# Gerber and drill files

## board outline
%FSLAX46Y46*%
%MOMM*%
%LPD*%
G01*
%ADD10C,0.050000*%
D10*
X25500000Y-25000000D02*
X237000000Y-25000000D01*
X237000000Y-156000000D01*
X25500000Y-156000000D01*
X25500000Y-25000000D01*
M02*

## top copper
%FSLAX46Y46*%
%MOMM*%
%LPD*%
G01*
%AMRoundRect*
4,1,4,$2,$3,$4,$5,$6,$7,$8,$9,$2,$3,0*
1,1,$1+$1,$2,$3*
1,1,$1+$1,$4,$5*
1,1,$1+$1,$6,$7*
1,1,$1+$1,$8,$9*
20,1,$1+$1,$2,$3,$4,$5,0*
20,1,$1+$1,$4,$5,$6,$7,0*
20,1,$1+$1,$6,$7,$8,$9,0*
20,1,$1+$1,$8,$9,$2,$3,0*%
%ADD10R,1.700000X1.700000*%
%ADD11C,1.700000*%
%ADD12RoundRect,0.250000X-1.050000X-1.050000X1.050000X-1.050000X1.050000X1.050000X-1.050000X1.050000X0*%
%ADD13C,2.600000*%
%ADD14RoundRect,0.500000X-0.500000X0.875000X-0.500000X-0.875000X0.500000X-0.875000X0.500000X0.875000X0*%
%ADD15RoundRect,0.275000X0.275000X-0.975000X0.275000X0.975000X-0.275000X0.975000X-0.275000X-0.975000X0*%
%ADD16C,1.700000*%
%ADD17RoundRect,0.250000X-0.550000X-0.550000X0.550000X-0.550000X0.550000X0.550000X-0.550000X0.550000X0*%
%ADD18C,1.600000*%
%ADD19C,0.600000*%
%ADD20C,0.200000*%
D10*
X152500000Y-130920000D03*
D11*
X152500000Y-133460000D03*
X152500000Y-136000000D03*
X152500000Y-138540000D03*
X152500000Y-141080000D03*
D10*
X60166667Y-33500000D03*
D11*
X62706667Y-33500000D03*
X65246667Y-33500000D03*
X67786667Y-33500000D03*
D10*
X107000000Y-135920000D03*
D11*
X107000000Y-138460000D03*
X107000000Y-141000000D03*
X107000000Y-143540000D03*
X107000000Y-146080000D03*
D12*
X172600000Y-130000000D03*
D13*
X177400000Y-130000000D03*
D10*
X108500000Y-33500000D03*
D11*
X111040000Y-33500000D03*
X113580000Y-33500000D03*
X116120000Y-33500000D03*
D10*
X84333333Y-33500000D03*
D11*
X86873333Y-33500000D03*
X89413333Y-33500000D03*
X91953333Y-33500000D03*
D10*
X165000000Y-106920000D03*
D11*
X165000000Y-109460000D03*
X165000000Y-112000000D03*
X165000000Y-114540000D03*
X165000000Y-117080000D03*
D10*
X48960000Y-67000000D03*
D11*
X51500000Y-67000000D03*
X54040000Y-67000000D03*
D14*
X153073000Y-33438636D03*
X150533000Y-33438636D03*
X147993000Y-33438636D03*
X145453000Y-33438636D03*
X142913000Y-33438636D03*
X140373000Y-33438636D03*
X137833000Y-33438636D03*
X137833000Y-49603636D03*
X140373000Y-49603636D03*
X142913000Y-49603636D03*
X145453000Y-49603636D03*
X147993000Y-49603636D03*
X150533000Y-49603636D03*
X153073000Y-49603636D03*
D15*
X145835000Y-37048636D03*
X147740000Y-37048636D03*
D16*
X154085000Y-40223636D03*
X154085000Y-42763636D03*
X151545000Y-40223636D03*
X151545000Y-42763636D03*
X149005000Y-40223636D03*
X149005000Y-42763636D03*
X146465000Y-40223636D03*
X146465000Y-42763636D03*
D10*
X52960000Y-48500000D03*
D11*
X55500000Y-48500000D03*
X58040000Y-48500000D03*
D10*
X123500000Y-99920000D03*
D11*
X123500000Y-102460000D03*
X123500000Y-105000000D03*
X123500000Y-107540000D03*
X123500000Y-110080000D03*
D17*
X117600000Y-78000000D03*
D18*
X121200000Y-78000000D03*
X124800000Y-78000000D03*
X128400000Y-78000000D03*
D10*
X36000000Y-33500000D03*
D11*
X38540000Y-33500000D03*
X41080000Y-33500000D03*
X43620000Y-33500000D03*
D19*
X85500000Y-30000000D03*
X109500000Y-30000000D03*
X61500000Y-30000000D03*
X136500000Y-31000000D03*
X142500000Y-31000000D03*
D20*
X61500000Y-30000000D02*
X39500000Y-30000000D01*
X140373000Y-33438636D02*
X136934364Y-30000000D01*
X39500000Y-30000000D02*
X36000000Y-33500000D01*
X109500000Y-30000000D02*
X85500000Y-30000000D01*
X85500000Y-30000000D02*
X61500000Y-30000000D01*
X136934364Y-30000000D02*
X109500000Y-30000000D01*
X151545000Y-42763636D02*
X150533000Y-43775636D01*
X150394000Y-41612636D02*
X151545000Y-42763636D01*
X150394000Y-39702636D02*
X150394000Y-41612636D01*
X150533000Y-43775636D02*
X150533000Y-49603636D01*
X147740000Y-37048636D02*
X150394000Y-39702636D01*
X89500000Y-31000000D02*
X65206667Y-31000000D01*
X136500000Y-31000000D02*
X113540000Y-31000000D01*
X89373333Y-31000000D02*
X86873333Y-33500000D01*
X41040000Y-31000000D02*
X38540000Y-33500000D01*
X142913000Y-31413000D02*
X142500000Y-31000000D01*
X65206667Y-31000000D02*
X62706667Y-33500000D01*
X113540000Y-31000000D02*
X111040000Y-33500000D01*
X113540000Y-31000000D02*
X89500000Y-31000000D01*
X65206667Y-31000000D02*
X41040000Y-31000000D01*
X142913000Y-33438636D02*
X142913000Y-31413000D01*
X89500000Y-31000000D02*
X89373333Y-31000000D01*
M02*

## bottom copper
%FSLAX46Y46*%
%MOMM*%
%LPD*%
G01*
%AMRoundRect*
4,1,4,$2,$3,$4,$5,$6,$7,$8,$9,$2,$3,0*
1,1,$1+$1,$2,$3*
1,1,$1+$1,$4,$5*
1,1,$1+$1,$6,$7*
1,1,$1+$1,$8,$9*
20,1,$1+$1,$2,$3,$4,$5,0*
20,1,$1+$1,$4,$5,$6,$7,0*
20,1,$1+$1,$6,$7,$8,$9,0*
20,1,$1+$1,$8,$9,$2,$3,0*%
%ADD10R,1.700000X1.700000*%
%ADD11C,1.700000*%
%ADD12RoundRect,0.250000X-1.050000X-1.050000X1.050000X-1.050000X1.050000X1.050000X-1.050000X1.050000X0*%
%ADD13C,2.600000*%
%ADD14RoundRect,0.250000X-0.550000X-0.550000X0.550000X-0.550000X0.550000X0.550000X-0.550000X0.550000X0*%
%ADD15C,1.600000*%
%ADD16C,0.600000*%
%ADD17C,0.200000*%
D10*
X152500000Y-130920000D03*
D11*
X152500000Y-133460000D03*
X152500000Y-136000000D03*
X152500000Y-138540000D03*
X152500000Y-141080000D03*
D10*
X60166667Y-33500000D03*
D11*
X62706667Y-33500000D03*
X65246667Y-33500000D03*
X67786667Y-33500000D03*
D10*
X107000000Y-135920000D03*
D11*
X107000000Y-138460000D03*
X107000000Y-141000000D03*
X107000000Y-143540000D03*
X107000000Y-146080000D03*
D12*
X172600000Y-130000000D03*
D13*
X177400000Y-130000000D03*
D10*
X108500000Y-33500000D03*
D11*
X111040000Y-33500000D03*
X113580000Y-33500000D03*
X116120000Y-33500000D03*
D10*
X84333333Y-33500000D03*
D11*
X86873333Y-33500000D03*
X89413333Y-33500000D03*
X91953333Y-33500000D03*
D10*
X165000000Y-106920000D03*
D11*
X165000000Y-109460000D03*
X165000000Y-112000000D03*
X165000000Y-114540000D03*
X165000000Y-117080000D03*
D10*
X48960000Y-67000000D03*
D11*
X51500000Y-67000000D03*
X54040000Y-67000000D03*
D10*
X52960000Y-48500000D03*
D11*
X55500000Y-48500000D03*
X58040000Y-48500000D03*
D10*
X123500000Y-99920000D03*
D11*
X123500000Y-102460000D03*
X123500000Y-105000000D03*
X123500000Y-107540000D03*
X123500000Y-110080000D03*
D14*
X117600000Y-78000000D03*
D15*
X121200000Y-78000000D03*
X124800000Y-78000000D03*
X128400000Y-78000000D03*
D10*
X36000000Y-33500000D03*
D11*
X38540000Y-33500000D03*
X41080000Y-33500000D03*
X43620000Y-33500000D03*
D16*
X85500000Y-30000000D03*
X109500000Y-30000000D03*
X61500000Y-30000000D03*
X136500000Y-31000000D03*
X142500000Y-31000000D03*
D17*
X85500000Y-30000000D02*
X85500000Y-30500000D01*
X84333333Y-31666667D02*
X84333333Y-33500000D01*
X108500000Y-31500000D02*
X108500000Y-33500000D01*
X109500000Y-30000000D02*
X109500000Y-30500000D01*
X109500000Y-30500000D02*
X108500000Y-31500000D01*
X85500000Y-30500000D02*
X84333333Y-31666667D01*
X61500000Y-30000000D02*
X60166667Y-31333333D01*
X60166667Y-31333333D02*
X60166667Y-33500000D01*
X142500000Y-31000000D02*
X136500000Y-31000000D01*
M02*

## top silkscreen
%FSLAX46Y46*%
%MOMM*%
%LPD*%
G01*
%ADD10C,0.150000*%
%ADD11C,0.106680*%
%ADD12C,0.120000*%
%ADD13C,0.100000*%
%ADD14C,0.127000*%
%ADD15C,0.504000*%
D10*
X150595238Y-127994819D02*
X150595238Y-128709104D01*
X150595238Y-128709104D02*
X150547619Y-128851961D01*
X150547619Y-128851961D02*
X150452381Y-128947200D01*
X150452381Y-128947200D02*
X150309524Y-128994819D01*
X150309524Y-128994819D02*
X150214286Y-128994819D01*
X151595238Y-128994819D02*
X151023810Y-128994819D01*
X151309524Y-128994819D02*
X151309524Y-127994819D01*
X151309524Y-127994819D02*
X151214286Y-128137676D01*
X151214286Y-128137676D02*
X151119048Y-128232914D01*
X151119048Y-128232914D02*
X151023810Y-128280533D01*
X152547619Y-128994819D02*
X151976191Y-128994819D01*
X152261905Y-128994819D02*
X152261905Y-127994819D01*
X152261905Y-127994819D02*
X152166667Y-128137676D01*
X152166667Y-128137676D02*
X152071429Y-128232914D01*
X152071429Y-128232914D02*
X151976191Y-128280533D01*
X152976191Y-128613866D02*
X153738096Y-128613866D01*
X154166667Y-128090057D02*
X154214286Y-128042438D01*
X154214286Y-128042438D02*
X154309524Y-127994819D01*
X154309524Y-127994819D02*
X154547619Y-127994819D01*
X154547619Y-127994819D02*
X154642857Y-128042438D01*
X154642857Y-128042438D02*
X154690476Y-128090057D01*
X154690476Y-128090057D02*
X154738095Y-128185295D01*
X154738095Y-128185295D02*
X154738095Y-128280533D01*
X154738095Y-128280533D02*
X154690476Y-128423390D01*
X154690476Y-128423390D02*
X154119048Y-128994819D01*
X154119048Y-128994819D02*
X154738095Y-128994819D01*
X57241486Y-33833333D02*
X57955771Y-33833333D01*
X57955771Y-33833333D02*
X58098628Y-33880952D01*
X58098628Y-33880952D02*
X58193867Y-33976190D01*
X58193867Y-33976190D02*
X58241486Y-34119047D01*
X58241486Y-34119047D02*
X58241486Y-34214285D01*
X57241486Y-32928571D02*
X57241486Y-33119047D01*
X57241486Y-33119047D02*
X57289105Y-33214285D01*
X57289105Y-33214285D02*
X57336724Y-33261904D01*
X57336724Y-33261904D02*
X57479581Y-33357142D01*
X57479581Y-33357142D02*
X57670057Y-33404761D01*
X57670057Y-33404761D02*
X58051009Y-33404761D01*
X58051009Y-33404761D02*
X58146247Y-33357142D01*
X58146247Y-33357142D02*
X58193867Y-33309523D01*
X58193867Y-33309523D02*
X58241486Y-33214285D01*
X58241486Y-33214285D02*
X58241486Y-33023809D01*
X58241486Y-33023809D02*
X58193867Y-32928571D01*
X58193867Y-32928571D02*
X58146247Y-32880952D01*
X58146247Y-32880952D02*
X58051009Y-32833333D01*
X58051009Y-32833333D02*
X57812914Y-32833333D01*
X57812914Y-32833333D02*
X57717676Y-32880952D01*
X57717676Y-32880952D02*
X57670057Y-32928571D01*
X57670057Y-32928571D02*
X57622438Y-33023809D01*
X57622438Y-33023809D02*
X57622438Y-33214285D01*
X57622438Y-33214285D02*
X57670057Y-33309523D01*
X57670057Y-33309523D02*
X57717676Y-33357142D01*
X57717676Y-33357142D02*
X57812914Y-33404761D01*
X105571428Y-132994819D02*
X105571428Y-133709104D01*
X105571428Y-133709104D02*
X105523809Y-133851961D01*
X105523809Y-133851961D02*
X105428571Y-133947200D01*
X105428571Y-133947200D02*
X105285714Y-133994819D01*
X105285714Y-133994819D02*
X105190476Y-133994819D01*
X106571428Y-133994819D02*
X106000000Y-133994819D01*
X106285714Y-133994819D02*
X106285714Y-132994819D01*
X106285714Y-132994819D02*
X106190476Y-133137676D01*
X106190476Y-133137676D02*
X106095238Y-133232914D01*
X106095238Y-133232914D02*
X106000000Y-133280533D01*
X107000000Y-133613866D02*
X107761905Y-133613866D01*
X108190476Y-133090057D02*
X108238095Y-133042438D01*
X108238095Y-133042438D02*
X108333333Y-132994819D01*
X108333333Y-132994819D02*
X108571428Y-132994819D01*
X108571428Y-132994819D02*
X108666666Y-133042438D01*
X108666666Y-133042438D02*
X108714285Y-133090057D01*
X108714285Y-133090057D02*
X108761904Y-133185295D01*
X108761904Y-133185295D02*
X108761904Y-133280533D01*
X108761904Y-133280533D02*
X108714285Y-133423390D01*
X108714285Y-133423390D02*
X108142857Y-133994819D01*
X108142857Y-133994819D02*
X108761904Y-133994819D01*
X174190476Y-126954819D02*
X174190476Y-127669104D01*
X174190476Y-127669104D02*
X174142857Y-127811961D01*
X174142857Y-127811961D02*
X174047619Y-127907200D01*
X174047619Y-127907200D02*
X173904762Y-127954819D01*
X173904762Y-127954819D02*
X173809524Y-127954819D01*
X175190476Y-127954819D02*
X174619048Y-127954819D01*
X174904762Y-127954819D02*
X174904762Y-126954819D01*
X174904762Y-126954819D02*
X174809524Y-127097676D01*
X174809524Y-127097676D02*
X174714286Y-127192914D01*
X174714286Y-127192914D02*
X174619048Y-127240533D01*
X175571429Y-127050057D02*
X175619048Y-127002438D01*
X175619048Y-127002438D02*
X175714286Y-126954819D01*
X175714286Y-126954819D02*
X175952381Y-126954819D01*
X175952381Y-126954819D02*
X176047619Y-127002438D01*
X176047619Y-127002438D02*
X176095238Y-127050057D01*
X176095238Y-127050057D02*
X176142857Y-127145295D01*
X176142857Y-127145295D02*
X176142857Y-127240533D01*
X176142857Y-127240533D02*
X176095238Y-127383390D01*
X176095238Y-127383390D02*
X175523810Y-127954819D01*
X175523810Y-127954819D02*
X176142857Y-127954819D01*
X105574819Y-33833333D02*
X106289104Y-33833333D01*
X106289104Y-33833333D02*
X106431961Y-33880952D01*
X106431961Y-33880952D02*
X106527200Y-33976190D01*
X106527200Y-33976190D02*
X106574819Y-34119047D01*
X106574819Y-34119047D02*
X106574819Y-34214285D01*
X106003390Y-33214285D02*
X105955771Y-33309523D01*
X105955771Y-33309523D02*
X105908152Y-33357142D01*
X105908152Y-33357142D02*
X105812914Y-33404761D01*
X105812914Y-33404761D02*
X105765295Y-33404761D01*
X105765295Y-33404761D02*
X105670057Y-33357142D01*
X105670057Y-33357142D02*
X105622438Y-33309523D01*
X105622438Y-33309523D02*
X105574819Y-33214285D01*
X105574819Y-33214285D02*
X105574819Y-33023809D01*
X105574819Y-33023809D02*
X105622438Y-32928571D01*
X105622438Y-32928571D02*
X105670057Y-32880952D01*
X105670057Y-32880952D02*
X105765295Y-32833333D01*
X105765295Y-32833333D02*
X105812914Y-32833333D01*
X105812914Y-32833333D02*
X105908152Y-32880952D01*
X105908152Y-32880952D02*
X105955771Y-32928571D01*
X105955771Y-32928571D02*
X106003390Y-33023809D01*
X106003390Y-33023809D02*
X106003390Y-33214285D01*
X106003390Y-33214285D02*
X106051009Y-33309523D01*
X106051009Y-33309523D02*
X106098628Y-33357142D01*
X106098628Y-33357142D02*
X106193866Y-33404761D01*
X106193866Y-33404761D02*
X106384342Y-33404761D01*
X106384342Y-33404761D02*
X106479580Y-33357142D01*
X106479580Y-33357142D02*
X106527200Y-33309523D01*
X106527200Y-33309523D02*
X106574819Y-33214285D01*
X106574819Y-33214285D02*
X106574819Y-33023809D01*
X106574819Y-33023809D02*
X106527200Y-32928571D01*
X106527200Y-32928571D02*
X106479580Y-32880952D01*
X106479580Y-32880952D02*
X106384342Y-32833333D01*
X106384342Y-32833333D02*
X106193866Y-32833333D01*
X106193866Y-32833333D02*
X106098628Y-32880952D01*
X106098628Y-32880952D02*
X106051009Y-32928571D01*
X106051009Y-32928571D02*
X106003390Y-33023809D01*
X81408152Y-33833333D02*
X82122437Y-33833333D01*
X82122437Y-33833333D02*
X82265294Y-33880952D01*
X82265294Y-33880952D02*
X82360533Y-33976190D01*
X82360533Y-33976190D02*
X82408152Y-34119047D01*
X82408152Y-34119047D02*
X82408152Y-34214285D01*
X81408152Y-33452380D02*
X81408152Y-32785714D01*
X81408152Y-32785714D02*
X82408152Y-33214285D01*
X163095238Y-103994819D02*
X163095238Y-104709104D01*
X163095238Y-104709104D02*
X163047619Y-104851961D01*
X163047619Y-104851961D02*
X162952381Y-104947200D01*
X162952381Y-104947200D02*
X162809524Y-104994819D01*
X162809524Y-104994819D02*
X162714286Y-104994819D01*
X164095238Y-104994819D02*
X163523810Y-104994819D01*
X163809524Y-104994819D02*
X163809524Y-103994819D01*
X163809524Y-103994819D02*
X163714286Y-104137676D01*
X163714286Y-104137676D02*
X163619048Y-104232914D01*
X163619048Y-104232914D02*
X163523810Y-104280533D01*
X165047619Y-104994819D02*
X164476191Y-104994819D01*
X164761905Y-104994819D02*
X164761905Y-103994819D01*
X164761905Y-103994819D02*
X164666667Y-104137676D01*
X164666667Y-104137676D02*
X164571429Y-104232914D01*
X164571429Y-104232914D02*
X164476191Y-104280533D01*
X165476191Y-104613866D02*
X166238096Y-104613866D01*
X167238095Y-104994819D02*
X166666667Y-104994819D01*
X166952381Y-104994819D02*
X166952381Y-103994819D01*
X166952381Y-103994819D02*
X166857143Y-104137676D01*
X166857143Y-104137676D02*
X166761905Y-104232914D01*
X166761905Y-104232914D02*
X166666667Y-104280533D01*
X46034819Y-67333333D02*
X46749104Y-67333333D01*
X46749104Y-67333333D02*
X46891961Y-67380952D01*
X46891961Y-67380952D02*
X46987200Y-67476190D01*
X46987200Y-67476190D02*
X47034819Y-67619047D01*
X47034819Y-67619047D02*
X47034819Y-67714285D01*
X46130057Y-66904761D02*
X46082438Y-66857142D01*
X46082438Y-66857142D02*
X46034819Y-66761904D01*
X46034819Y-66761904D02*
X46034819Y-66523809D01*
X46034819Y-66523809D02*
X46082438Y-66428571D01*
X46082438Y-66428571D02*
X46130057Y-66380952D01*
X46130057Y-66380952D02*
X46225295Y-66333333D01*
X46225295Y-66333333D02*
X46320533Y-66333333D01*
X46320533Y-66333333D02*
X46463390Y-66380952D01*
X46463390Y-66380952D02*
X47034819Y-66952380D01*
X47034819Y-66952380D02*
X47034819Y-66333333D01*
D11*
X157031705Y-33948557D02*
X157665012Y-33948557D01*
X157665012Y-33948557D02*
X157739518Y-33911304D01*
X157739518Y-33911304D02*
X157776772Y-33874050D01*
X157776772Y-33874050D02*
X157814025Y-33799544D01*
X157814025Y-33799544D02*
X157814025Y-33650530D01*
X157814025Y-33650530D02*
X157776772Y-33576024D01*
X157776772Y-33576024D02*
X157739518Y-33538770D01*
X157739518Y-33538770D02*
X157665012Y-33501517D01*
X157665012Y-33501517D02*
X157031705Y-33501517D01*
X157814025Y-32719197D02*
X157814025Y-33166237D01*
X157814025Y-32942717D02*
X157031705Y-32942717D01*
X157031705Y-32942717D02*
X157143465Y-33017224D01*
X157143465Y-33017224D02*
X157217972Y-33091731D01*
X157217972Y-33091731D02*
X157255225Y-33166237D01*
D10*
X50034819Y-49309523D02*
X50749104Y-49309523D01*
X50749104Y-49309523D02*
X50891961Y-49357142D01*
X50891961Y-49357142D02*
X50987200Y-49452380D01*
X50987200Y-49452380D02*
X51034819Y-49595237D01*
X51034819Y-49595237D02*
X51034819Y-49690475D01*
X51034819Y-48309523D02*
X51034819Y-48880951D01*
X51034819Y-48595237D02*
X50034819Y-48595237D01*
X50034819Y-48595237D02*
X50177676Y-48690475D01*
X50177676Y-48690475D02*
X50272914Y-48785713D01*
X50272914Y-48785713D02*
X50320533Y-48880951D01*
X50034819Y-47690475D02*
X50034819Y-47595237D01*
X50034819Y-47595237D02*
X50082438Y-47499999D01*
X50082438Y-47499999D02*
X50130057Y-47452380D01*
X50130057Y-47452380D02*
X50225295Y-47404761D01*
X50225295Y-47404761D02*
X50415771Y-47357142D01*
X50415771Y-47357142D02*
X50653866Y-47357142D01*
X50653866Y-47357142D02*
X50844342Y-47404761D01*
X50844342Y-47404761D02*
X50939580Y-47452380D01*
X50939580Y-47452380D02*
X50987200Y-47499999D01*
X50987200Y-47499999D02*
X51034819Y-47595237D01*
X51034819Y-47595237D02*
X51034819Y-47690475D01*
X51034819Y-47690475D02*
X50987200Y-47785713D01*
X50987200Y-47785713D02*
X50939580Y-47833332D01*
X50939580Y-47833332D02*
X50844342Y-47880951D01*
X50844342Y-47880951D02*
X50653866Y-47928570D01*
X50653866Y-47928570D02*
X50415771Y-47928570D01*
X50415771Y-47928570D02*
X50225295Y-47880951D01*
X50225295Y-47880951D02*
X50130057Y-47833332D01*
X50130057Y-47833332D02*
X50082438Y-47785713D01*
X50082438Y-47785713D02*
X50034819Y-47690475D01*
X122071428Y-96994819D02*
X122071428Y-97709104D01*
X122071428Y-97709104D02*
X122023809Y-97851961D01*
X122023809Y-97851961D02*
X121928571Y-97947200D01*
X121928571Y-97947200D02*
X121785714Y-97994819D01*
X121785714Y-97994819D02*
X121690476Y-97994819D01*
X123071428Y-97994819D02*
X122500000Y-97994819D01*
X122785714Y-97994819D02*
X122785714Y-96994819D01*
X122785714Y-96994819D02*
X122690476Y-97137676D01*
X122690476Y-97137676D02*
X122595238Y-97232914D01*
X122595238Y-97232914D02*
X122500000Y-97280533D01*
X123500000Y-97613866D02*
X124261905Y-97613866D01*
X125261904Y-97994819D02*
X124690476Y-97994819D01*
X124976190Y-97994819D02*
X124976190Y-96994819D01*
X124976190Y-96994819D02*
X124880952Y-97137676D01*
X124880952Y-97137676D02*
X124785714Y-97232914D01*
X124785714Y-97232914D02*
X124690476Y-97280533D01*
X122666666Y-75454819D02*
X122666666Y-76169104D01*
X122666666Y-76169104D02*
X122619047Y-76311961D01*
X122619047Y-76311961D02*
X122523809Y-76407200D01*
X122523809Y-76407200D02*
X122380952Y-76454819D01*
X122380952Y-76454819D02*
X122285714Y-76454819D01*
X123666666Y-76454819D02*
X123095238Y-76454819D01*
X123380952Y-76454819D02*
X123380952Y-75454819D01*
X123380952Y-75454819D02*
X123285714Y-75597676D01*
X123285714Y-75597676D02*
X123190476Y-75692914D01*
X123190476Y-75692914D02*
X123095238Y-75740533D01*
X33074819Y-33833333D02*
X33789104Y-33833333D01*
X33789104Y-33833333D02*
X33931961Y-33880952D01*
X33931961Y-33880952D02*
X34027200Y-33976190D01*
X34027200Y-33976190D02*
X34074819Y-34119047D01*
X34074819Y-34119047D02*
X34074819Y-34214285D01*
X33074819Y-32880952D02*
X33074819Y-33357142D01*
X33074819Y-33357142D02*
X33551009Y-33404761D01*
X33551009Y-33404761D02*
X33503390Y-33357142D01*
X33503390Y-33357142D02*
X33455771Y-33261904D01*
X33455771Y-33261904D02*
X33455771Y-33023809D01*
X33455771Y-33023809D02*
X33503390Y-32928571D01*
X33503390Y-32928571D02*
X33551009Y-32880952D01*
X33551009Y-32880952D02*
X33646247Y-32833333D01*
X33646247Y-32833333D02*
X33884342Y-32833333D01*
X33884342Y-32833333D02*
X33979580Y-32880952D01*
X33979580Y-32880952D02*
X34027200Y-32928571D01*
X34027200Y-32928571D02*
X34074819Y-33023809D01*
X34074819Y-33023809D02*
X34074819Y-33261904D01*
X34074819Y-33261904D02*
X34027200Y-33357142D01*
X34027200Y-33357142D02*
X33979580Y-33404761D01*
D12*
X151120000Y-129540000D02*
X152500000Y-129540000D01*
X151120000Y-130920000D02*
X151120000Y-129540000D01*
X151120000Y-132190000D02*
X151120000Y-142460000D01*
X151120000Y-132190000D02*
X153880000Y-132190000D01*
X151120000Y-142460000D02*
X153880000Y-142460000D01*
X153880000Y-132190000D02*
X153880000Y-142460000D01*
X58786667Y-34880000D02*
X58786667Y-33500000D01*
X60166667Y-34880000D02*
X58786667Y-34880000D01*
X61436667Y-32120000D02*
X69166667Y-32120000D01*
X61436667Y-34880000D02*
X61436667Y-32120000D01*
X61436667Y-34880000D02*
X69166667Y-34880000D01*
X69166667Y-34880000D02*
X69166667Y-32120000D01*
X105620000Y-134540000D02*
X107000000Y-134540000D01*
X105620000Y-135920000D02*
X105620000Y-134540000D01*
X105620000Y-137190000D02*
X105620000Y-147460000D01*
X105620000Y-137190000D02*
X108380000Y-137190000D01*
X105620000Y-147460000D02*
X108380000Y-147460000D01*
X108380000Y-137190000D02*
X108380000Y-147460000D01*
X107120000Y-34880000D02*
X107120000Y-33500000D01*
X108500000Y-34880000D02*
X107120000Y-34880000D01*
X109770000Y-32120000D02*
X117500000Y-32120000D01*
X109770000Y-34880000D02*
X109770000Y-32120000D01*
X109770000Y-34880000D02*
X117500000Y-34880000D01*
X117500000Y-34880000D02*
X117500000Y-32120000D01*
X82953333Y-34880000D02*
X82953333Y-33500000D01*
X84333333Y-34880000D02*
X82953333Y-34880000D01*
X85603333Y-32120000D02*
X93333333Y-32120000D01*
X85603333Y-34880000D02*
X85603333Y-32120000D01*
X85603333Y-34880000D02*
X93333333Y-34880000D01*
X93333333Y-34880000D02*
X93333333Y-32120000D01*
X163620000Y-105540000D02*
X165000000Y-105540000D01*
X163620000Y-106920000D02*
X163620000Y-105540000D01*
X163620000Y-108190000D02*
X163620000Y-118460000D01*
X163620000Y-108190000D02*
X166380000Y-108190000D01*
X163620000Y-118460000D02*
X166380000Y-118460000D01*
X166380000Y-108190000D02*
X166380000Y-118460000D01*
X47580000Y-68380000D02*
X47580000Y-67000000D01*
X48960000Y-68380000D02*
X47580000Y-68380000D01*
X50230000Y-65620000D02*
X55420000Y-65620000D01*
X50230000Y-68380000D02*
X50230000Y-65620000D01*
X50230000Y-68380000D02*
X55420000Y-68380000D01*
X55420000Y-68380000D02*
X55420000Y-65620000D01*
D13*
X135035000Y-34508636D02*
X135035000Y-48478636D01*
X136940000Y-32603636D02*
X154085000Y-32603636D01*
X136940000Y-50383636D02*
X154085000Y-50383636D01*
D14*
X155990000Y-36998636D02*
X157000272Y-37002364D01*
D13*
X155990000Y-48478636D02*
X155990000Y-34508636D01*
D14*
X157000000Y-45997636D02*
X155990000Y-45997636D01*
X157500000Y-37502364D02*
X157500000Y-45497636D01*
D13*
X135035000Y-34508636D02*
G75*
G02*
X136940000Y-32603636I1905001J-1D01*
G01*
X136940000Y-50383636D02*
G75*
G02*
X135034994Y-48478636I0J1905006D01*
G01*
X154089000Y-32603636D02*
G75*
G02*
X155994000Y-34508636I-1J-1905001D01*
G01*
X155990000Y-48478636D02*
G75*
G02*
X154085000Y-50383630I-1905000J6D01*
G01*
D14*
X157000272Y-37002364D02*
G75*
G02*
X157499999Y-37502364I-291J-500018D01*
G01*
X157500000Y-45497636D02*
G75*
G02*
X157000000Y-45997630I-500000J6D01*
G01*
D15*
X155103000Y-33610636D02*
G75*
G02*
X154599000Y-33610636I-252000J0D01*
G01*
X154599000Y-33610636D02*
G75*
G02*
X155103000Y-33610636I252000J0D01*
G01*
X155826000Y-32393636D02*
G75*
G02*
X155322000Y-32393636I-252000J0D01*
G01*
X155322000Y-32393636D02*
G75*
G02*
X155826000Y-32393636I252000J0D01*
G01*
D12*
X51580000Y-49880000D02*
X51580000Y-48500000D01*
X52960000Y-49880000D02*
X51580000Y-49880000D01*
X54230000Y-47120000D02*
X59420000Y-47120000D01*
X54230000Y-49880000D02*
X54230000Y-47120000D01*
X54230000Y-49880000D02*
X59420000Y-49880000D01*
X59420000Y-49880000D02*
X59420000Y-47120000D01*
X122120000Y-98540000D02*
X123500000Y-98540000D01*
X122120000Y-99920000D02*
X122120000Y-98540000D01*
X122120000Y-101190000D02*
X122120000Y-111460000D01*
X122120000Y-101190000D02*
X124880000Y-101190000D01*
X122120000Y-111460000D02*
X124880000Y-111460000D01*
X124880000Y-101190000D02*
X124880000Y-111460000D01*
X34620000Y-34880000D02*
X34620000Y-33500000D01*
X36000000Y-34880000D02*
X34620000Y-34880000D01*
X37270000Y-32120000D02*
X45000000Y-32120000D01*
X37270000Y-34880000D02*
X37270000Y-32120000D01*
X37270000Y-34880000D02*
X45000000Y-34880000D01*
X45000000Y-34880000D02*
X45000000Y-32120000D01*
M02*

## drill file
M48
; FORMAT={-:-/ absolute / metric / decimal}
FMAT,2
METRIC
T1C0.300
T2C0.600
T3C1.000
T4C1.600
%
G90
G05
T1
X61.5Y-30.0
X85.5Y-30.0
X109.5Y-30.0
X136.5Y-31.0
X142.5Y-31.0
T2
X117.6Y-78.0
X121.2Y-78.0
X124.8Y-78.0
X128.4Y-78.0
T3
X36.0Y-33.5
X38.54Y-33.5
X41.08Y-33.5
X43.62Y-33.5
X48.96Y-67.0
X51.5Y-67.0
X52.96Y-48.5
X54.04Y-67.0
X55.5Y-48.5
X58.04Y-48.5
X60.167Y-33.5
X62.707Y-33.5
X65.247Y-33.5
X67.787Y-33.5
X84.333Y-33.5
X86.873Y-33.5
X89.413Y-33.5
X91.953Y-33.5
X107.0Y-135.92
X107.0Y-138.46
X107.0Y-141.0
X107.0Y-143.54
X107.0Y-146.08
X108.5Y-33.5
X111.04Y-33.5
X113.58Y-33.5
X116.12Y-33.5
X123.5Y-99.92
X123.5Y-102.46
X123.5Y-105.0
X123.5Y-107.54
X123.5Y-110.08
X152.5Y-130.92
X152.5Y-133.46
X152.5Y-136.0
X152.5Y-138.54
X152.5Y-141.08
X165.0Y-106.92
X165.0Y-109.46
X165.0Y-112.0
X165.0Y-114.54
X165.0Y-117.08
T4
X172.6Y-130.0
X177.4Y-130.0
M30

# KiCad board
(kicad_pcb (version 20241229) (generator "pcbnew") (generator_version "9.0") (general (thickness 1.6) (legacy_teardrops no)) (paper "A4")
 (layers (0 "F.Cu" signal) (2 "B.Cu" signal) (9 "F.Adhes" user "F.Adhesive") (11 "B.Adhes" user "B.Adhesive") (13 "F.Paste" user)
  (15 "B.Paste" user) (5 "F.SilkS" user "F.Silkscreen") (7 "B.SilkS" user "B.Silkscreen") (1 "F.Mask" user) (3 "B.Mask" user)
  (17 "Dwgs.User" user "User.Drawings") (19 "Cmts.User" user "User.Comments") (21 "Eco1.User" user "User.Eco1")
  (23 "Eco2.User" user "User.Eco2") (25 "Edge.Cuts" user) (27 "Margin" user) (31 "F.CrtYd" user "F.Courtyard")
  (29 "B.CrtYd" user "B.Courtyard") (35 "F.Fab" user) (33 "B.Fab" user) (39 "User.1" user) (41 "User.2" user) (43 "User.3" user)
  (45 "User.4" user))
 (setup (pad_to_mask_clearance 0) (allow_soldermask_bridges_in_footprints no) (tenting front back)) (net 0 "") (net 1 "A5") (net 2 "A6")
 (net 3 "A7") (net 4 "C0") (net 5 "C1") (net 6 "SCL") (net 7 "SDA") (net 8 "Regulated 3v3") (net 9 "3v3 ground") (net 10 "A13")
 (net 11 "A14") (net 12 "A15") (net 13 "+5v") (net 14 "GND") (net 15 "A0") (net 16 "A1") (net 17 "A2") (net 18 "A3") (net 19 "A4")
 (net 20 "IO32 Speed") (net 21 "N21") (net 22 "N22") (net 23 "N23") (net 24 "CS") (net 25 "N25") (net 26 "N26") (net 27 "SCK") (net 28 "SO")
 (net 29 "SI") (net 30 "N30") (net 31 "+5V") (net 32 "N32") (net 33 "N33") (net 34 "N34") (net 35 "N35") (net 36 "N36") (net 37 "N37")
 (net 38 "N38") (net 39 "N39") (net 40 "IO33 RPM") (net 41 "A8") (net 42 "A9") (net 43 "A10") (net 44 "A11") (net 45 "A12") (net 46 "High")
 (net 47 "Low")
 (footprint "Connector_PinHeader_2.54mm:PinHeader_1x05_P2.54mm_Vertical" (layer "F.Cu") (at 152.5 130.92)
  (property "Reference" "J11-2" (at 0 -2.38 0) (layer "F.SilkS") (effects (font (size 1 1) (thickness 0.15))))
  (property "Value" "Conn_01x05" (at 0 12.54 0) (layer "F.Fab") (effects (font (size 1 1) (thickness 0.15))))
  (fp_line (start -1.38 -1.38) (end 0 -1.38) (stroke (width 0.12) (type solid)) (layer "F.SilkS"))
  (fp_line (start -1.38 0) (end -1.38 -1.38) (stroke (width 0.12) (type solid)) (layer "F.SilkS"))
  (fp_line (start -1.38 1.27) (end -1.38 11.54) (stroke (width 0.12) (type solid)) (layer "F.SilkS"))
  (fp_line (start -1.38 1.27) (end 1.38 1.27) (stroke (width 0.12) (type solid)) (layer "F.SilkS"))
  (fp_line (start -1.38 11.54) (end 1.38 11.54) (stroke (width 0.12) (type solid)) (layer "F.SilkS"))
  (fp_line (start 1.38 1.27) (end 1.38 11.54) (stroke (width 0.12) (type solid)) (layer "F.SilkS"))
  (pad "1" thru_hole rect (at 0 0) (size 1.7 1.7) (drill 1) (layers "*.Cu" "*.Mask") (remove_unused_layers no) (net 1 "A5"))
  (pad "2" thru_hole circle (at 0 2.54) (size 1.7 1.7) (drill 1) (layers "*.Cu" "*.Mask") (remove_unused_layers no) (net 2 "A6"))
  (pad "3" thru_hole circle (at 0 5.08) (size 1.7 1.7) (drill 1) (layers "*.Cu" "*.Mask") (remove_unused_layers no) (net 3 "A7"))
  (pad "4" thru_hole circle (at 0 7.62) (size 1.7 1.7) (drill 1) (layers "*.Cu" "*.Mask") (remove_unused_layers no) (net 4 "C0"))
  (pad "5" thru_hole circle (at 0 10.16) (size 1.7 1.7) (drill 1) (layers "*.Cu" "*.Mask") (remove_unused_layers no) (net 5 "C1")))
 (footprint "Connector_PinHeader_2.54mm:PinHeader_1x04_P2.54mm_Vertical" (layer "F.Cu") (at 60.166667 33.5 90)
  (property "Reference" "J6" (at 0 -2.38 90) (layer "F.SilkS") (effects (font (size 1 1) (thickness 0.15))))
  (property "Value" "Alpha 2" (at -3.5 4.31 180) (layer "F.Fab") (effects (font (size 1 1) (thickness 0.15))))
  (fp_line (start -1.38 -1.38) (end 0 -1.38) (stroke (width 0.12) (type solid)) (layer "F.SilkS"))
  (fp_line (start -1.38 0) (end -1.38 -1.38) (stroke (width 0.12) (type solid)) (layer "F.SilkS"))
  (fp_line (start 1.38 1.27) (end 1.38 9) (stroke (width 0.12) (type solid)) (layer "F.SilkS"))
  (fp_line (start -1.38 1.27) (end 1.38 1.27) (stroke (width 0.12) (type solid)) (layer "F.SilkS"))
  (fp_line (start -1.38 1.27) (end -1.38 9) (stroke (width 0.12) (type solid)) (layer "F.SilkS"))
  (fp_line (start -1.38 9) (end 1.38 9) (stroke (width 0.12) (type solid)) (layer "F.SilkS"))
  (pad "1" thru_hole rect (at 0 0 90) (size 1.7 1.7) (drill 1) (layers "*.Cu" "*.Mask") (remove_unused_layers no) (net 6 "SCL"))
  (pad "2" thru_hole circle (at 0 2.54 90) (size 1.7 1.7) (drill 1) (layers "*.Cu" "*.Mask") (remove_unused_layers no) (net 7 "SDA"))
  (pad "3" thru_hole circle (at 0 5.08 90) (size 1.7 1.7) (drill 1) (layers "*.Cu" "*.Mask") (remove_unused_layers no)
   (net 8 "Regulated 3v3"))
  (pad "4" thru_hole circle (at 0 7.62 90) (size 1.7 1.7) (drill 1) (layers "*.Cu" "*.Mask") (remove_unused_layers no) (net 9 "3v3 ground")))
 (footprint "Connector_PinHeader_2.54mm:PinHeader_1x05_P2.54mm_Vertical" (layer "F.Cu") (at 107 135.92)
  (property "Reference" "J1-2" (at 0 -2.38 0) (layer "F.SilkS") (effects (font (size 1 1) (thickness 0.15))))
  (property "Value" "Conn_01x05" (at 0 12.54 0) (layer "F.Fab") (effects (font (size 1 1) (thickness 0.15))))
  (fp_line (start -1.38 -1.38) (end 0 -1.38) (stroke (width 0.12) (type solid)) (layer "F.SilkS"))
  (fp_line (start -1.38 0) (end -1.38 -1.38) (stroke (width 0.12) (type solid)) (layer "F.SilkS"))
  (fp_line (start -1.38 1.27) (end -1.38 11.54) (stroke (width 0.12) (type solid)) (layer "F.SilkS"))
  (fp_line (start -1.38 1.27) (end 1.38 1.27) (stroke (width 0.12) (type solid)) (layer "F.SilkS"))
  (fp_line (start -1.38 11.54) (end 1.38 11.54) (stroke (width 0.12) (type solid)) (layer "F.SilkS"))
  (fp_line (start 1.38 1.27) (end 1.38 11.54) (stroke (width 0.12) (type solid)) (layer "F.SilkS"))
  (pad "1" thru_hole rect (at 0 0) (size 1.7 1.7) (drill 1) (layers "*.Cu" "*.Mask") (remove_unused_layers no) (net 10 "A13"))
  (pad "2" thru_hole circle (at 0 2.54) (size 1.7 1.7) (drill 1) (layers "*.Cu" "*.Mask") (remove_unused_layers no) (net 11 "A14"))
  (pad "3" thru_hole circle (at 0 5.08) (size 1.7 1.7) (drill 1) (layers "*.Cu" "*.Mask") (remove_unused_layers no) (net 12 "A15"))
  (pad "4" thru_hole circle (at 0 7.62) (size 1.7 1.7) (drill 1) (layers "*.Cu" "*.Mask") (remove_unused_layers no) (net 4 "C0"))
  (pad "5" thru_hole circle (at 0 10.16) (size 1.7 1.7) (drill 1) (layers "*.Cu" "*.Mask") (remove_unused_layers no) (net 5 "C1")))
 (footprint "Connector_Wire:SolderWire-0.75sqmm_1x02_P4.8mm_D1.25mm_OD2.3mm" (layer "F.Cu") (at 172.6 130)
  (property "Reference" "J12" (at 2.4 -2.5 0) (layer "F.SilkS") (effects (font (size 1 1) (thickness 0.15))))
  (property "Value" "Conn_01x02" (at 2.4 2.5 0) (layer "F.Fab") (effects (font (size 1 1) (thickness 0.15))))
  (pad "1" thru_hole roundrect (at 0 0) (size 2.6 2.6) (drill 1.6) (layers "*.Cu" "*.Mask") (remove_unused_layers no)
   (roundrect_rratio 0.096154) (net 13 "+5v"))
  (pad "2" thru_hole circle (at 4.8 0) (size 2.6 2.6) (drill 1.6) (layers "*.Cu" "*.Mask") (remove_unused_layers no) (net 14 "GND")))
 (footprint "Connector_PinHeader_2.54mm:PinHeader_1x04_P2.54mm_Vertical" (layer "F.Cu") (at 108.5 33.5 90)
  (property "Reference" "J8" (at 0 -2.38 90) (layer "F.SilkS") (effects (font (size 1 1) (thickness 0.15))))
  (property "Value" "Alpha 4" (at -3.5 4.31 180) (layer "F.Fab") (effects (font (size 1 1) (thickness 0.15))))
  (fp_line (start -1.38 -1.38) (end 0 -1.38) (stroke (width 0.12) (type solid)) (layer "F.SilkS"))
  (fp_line (start -1.38 0) (end -1.38 -1.38) (stroke (width 0.12) (type solid)) (layer "F.SilkS"))
  (fp_line (start 1.38 1.27) (end 1.38 9) (stroke (width 0.12) (type solid)) (layer "F.SilkS"))
  (fp_line (start -1.38 1.27) (end 1.38 1.27) (stroke (width 0.12) (type solid)) (layer "F.SilkS"))
  (fp_line (start -1.38 1.27) (end -1.38 9) (stroke (width 0.12) (type solid)) (layer "F.SilkS"))
  (fp_line (start -1.38 9) (end 1.38 9) (stroke (width 0.12) (type solid)) (layer "F.SilkS"))
  (pad "1" thru_hole rect (at 0 0 90) (size 1.7 1.7) (drill 1) (layers "*.Cu" "*.Mask") (remove_unused_layers no) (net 6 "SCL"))
  (pad "2" thru_hole circle (at 0 2.54 90) (size 1.7 1.7) (drill 1) (layers "*.Cu" "*.Mask") (remove_unused_layers no) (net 7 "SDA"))
  (pad "3" thru_hole circle (at 0 5.08 90) (size 1.7 1.7) (drill 1) (layers "*.Cu" "*.Mask") (remove_unused_layers no)
   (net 8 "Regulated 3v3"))
  (pad "4" thru_hole circle (at 0 7.62 90) (size 1.7 1.7) (drill 1) (layers "*.Cu" "*.Mask") (remove_unused_layers no) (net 9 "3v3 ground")))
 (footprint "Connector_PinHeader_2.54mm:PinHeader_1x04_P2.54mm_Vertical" (layer "F.Cu") (at 84.333333 33.5 90)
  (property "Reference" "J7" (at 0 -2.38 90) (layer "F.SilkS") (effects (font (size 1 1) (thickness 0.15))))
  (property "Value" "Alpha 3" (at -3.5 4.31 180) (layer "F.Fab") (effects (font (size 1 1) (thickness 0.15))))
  (fp_line (start -1.38 -1.38) (end 0 -1.38) (stroke (width 0.12) (type solid)) (layer "F.SilkS"))
  (fp_line (start -1.38 0) (end -1.38 -1.38) (stroke (width 0.12) (type solid)) (layer "F.SilkS"))
  (fp_line (start 1.38 1.27) (end 1.38 9) (stroke (width 0.12) (type solid)) (layer "F.SilkS"))
  (fp_line (start -1.38 1.27) (end 1.38 1.27) (stroke (width 0.12) (type solid)) (layer "F.SilkS"))
  (fp_line (start -1.38 1.27) (end -1.38 9) (stroke (width 0.12) (type solid)) (layer "F.SilkS"))
  (fp_line (start -1.38 9) (end 1.38 9) (stroke (width 0.12) (type solid)) (layer "F.SilkS"))
  (pad "1" thru_hole rect (at 0 0 90) (size 1.7 1.7) (drill 1) (layers "*.Cu" "*.Mask") (remove_unused_layers no) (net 6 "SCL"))
  (pad "2" thru_hole circle (at 0 2.54 90) (size 1.7 1.7) (drill 1) (layers "*.Cu" "*.Mask") (remove_unused_layers no) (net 7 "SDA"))
  (pad "3" thru_hole circle (at 0 5.08 90) (size 1.7 1.7) (drill 1) (layers "*.Cu" "*.Mask") (remove_unused_layers no)
   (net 8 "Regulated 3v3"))
  (pad "4" thru_hole circle (at 0 7.62 90) (size 1.7 1.7) (drill 1) (layers "*.Cu" "*.Mask") (remove_unused_layers no) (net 9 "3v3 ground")))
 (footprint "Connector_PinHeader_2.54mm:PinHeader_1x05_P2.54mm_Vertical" (layer "F.Cu") (at 165 106.92)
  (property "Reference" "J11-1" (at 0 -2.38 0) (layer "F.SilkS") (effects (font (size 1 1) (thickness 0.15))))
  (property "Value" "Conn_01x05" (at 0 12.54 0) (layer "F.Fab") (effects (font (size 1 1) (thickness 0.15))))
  (fp_line (start -1.38 -1.38) (end 0 -1.38) (stroke (width 0.12) (type solid)) (layer "F.SilkS"))
  (fp_line (start -1.38 0) (end -1.38 -1.38) (stroke (width 0.12) (type solid)) (layer "F.SilkS"))
  (fp_line (start -1.38 1.27) (end -1.38 11.54) (stroke (width 0.12) (type solid)) (layer "F.SilkS"))
  (fp_line (start -1.38 1.27) (end 1.38 1.27) (stroke (width 0.12) (type solid)) (layer "F.SilkS"))
  (fp_line (start -1.38 11.54) (end 1.38 11.54) (stroke (width 0.12) (type solid)) (layer "F.SilkS"))
  (fp_line (start 1.38 1.27) (end 1.38 11.54) (stroke (width 0.12) (type solid)) (layer "F.SilkS"))
  (pad "1" thru_hole rect (at 0 0) (size 1.7 1.7) (drill 1) (layers "*.Cu" "*.Mask") (remove_unused_layers no) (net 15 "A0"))
  (pad "2" thru_hole circle (at 0 2.54) (size 1.7 1.7) (drill 1) (layers "*.Cu" "*.Mask") (remove_unused_layers no) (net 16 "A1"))
  (pad "3" thru_hole circle (at 0 5.08) (size 1.7 1.7) (drill 1) (layers "*.Cu" "*.Mask") (remove_unused_layers no) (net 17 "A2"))
  (pad "4" thru_hole circle (at 0 7.62) (size 1.7 1.7) (drill 1) (layers "*.Cu" "*.Mask") (remove_unused_layers no) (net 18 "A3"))
  (pad "5" thru_hole circle (at 0 10.16) (size 1.7 1.7) (drill 1) (layers "*.Cu" "*.Mask") (remove_unused_layers no) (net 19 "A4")))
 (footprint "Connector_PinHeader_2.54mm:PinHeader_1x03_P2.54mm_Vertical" (layer "F.Cu") (at 48.96 67 90)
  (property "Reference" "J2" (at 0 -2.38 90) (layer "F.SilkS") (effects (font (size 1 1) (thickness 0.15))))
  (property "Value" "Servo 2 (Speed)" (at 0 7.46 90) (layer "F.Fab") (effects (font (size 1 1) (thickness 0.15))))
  (fp_line (start -1.38 -1.38) (end 0 -1.38) (stroke (width 0.12) (type solid)) (layer "F.SilkS"))
  (fp_line (start -1.38 0) (end -1.38 -1.38) (stroke (width 0.12) (type solid)) (layer "F.SilkS"))
  (fp_line (start 1.38 1.27) (end 1.38 6.46) (stroke (width 0.12) (type solid)) (layer "F.SilkS"))
  (fp_line (start -1.38 1.27) (end 1.38 1.27) (stroke (width 0.12) (type solid)) (layer "F.SilkS"))
  (fp_line (start -1.38 1.27) (end -1.38 6.46) (stroke (width 0.12) (type solid)) (layer "F.SilkS"))
  (fp_line (start -1.38 6.46) (end 1.38 6.46) (stroke (width 0.12) (type solid)) (layer "F.SilkS"))
  (pad "1" thru_hole rect (at 0 0 90) (size 1.7 1.7) (drill 1) (layers "*.Cu" "*.Mask") (remove_unused_layers no) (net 14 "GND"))
  (pad "2" thru_hole circle (at 0 2.54 90) (size 1.7 1.7) (drill 1) (layers "*.Cu" "*.Mask") (remove_unused_layers no) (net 13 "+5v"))
  (pad "3" thru_hole circle (at 0 5.08 90) (size 1.7 1.7) (drill 1) (layers "*.Cu" "*.Mask") (remove_unused_layers no) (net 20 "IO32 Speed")))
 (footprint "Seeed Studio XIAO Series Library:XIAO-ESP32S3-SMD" (layer "F.Cu") (at 145.5 41.5 -90)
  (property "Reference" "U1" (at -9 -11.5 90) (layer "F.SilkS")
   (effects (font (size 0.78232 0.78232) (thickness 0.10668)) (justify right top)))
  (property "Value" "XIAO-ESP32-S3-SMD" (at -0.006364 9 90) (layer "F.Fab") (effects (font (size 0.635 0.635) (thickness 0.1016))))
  (fp_line (start -6.991364 10.465) (end 6.978636 10.465) (stroke (width 0.1) (type solid)) (layer "F.SilkS"))
  (fp_line (start -8.896364 8.56) (end -8.896364 -8.585) (stroke (width 0.1) (type solid)) (layer "F.SilkS"))
  (fp_line (start 8.883636 8.56) (end 8.883636 -8.585) (stroke (width 0.1) (type solid)) (layer "F.SilkS"))
  (fp_line (start -4.501364 -10.49) (end -4.497636 -11.500272) (stroke (width 0.127) (type solid)) (layer "F.SilkS"))
  (fp_line (start 6.978636 -10.49) (end -6.991364 -10.49) (stroke (width 0.1) (type solid)) (layer "F.SilkS"))
  (fp_line (start 4.497636 -11.5) (end 4.497636 -10.49) (stroke (width 0.127) (type solid)) (layer "F.SilkS"))
  (fp_line (start -3.997636 -12) (end 3.997636 -12) (stroke (width 0.127) (type solid)) (layer "F.SilkS"))
  (fp_arc (start -6.991364 10.465) (mid -8.338402 9.907038) (end -8.896364 8.56) (stroke (width 0.1) (type solid)) (layer "F.SilkS"))
  (fp_arc (start 8.883636 8.56) (mid 8.325674 9.907038) (end 6.978636 10.465) (stroke (width 0.1) (type solid)) (layer "F.SilkS"))
  (fp_arc (start -8.896364 -8.589) (mid -8.338402 -9.936038) (end -6.991364 -10.494) (stroke (width 0.1) (type solid)) (layer "F.SilkS"))
  (fp_arc (start 6.978636 -10.49) (mid 8.325674 -9.932038) (end 8.883636 -8.585) (stroke (width 0.1) (type solid)) (layer "F.SilkS"))
  (fp_arc (start -4.497636 -11.500272) (mid -4.351088 -11.853644) (end -3.997636 -12) (stroke (width 0.127) (type default))
   (layer "F.SilkS"))
  (fp_arc (start 3.997636 -12) (mid 4.351189 -11.853553) (end 4.497636 -11.5) (stroke (width 0.127) (type default)) (layer "F.SilkS"))
  (fp_circle (center -7.889364 -9.351) (end -7.889364 -9.605) (stroke (width 0.5) (type solid)) (fill yes) (layer "F.SilkS"))
  (fp_circle (center -9.106364 -10.074) (end -9.106364 -10.328) (stroke (width 0.5) (type solid)) (fill yes) (layer "F.SilkS"))
  (pad "1" smd roundrect (at -8.061364 -7.573 270) (size 2.75 2) (layers "F.Cu" "F.Mask" "F.Paste") (roundrect_rratio 0.25) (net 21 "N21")
   (solder_mask_margin 0.0508) (thermal_bridge_angle 45))
  (pad "2" smd roundrect (at -8.061364 -5.033 270) (size 2.75 2) (layers "F.Cu" "F.Mask" "F.Paste") (roundrect_rratio 0.25) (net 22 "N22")
   (solder_mask_margin 0.0508) (thermal_bridge_angle 45))
  (pad "3" smd roundrect (at -8.061364 -2.493 270) (size 2.75 2) (layers "F.Cu" "F.Mask" "F.Paste") (roundrect_rratio 0.25) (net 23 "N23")
   (solder_mask_margin 0.0508) (thermal_bridge_angle 45))
  (pad "4" smd roundrect (at -8.061364 0.047 270) (size 2.75 2) (layers "F.Cu" "F.Mask" "F.Paste") (roundrect_rratio 0.25) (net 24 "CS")
   (solder_mask_margin 0.0508) (thermal_bridge_angle 45))
  (pad "5" smd roundrect (at -8.061364 2.587 270) (size 2.75 2) (layers "F.Cu" "F.Mask" "F.Paste") (roundrect_rratio 0.25) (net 7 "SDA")
   (solder_mask_margin 0.0508) (thermal_bridge_angle 45))
  (pad "6" smd roundrect (at -8.061364 5.127 270) (size 2.75 2) (layers "F.Cu" "F.Mask" "F.Paste") (roundrect_rratio 0.25) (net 6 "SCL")
   (solder_mask_margin 0.0508) (thermal_bridge_angle 45))
  (pad "7" smd roundrect (at -8.061364 7.667 270) (size 2.75 2) (layers "F.Cu" "F.Mask" "F.Paste") (roundrect_rratio 0.25) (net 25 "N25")
   (solder_mask_margin 0.0508) (thermal_bridge_angle 45))
  (pad "8" smd roundrect (at 8.103636 7.667 270) (size 2.75 2) (layers "F.Cu" "F.Mask" "F.Paste") (roundrect_rratio 0.25) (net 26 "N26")
   (solder_mask_margin 0.0508) (thermal_bridge_angle 45))
  (pad "9" smd roundrect (at 8.103636 5.127 270) (size 2.75 2) (layers "F.Cu" "F.Mask" "F.Paste") (roundrect_rratio 0.25) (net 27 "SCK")
   (solder_mask_margin 0.0508) (thermal_bridge_angle 45))
  (pad "10" smd roundrect (at 8.103636 2.587 270) (size 2.75 2) (layers "F.Cu" "F.Mask" "F.Paste") (roundrect_rratio 0.25) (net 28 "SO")
   (solder_mask_margin 0.0508) (thermal_bridge_angle 45))
  (pad "11" smd roundrect (at 8.103636 0.047 270) (size 2.75 2) (layers "F.Cu" "F.Mask" "F.Paste") (roundrect_rratio 0.25) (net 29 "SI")
   (solder_mask_margin 0.0508) (thermal_bridge_angle 45))
  (pad "12" smd roundrect (at 8.103636 -2.493 270) (size 2.75 2) (layers "F.Cu" "F.Mask" "F.Paste") (roundrect_rratio 0.25) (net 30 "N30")
   (solder_mask_margin 0.0508) (thermal_bridge_angle 45))
  (pad "13" smd roundrect (at 8.103636 -5.033 270) (size 2.75 2) (layers "F.Cu" "F.Mask" "F.Paste") (roundrect_rratio 0.25) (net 14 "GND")
   (solder_mask_margin 0.0508) (thermal_bridge_angle 45))
  (pad "14" smd roundrect (at 8.103636 -7.573 270) (size 2.75 2) (layers "F.Cu" "F.Mask" "F.Paste") (roundrect_rratio 0.25) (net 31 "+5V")
   (solder_mask_margin 0.0508) (thermal_bridge_angle 45))
  (pad "15" smd roundrect (at -4.451364 -0.335 90) (size 2.5 1.1) (layers "F.Cu" "F.Mask" "F.Paste") (roundrect_rratio 0.25) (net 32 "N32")
   (solder_mask_margin 0.0508) (thermal_bridge_angle 45))
  (pad "16" smd roundrect (at -4.451364 -2.24 90) (size 2.5 1.1) (layers "F.Cu" "F.Mask" "F.Paste") (roundrect_rratio 0.25) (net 14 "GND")
   (solder_mask_margin 0.0508) (thermal_bridge_angle 45))
  (pad "17" smd circle (at -1.276364 -8.585 270) (size 1.7 1.7) (layers "F.Cu" "F.Mask" "F.Paste") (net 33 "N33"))
  (pad "18" smd circle (at 1.263636 -8.585 270) (size 1.7 1.7) (layers "F.Cu" "F.Mask" "F.Paste") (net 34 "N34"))
  (pad "19" smd circle (at -1.276364 -6.045 270) (size 1.7 1.7) (layers "F.Cu" "F.Mask" "F.Paste") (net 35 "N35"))
  (pad "20" smd circle (at 1.263636 -6.045 270) (size 1.7 1.7) (layers "F.Cu" "F.Mask" "F.Paste") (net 14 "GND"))
  (pad "21" smd circle (at -1.276364 -3.505 270) (size 1.7 1.7) (layers "F.Cu" "F.Mask" "F.Paste") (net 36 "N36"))
  (pad "22" smd circle (at 1.263636 -3.505 270) (size 1.7 1.7) (layers "F.Cu" "F.Mask" "F.Paste") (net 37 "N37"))
  (pad "23" smd circle (at -1.276364 -0.965 270) (size 1.7 1.7) (layers "F.Cu" "F.Mask" "F.Paste") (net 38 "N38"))
  (pad "24" smd circle (at 1.263636 -0.965 270) (size 1.7 1.7) (layers "F.Cu" "F.Mask" "F.Paste") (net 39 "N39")))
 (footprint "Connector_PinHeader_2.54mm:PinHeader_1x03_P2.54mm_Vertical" (layer "F.Cu") (at 52.96 48.5 90)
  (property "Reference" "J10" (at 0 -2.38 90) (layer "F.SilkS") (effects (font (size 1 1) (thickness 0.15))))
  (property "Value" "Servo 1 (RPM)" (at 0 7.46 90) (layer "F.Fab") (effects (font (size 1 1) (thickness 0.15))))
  (fp_line (start -1.38 -1.38) (end 0 -1.38) (stroke (width 0.12) (type solid)) (layer "F.SilkS"))
  (fp_line (start -1.38 0) (end -1.38 -1.38) (stroke (width 0.12) (type solid)) (layer "F.SilkS"))
  (fp_line (start 1.38 1.27) (end 1.38 6.46) (stroke (width 0.12) (type solid)) (layer "F.SilkS"))
  (fp_line (start -1.38 1.27) (end 1.38 1.27) (stroke (width 0.12) (type solid)) (layer "F.SilkS"))
  (fp_line (start -1.38 1.27) (end -1.38 6.46) (stroke (width 0.12) (type solid)) (layer "F.SilkS"))
  (fp_line (start -1.38 6.46) (end 1.38 6.46) (stroke (width 0.12) (type solid)) (layer "F.SilkS"))
  (pad "1" thru_hole rect (at 0 0 90) (size 1.7 1.7) (drill 1) (layers "*.Cu" "*.Mask") (remove_unused_layers no) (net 14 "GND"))
  (pad "2" thru_hole circle (at 0 2.54 90) (size 1.7 1.7) (drill 1) (layers "*.Cu" "*.Mask") (remove_unused_layers no) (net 13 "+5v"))
  (pad "3" thru_hole circle (at 0 5.08 90) (size 1.7 1.7) (drill 1) (layers "*.Cu" "*.Mask") (remove_unused_layers no) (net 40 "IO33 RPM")))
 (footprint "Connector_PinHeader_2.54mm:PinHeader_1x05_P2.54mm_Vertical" (layer "F.Cu") (at 123.5 99.92)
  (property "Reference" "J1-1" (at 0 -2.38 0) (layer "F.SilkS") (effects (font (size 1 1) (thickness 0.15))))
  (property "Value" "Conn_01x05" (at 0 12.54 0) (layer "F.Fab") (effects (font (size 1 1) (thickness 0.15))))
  (fp_line (start -1.38 -1.38) (end 0 -1.38) (stroke (width 0.12) (type solid)) (layer "F.SilkS"))
  (fp_line (start -1.38 0) (end -1.38 -1.38) (stroke (width 0.12) (type solid)) (layer "F.SilkS"))
  (fp_line (start -1.38 1.27) (end -1.38 11.54) (stroke (width 0.12) (type solid)) (layer "F.SilkS"))
  (fp_line (start -1.38 1.27) (end 1.38 1.27) (stroke (width 0.12) (type solid)) (layer "F.SilkS"))
  (fp_line (start -1.38 11.54) (end 1.38 11.54) (stroke (width 0.12) (type solid)) (layer "F.SilkS"))
  (fp_line (start 1.38 1.27) (end 1.38 11.54) (stroke (width 0.12) (type solid)) (layer "F.SilkS"))
  (pad "1" thru_hole rect (at 0 0) (size 1.7 1.7) (drill 1) (layers "*.Cu" "*.Mask") (remove_unused_layers no) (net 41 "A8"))
  (pad "2" thru_hole circle (at 0 2.54) (size 1.7 1.7) (drill 1) (layers "*.Cu" "*.Mask") (remove_unused_layers no) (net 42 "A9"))
  (pad "3" thru_hole circle (at 0 5.08) (size 1.7 1.7) (drill 1) (layers "*.Cu" "*.Mask") (remove_unused_layers no) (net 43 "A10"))
  (pad "4" thru_hole circle (at 0 7.62) (size 1.7 1.7) (drill 1) (layers "*.Cu" "*.Mask") (remove_unused_layers no) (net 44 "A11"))
  (pad "5" thru_hole circle (at 0 10.16) (size 1.7 1.7) (drill 1) (layers "*.Cu" "*.Mask") (remove_unused_layers no) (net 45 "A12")))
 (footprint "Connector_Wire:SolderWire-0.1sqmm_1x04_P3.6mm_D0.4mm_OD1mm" (layer "F.Cu") (at 117.6 78)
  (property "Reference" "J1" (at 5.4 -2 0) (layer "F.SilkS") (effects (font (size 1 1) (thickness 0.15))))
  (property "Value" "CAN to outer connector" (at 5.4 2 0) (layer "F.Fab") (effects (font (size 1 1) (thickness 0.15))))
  (pad "1" thru_hole roundrect (at 0 0) (size 1.6 1.6) (drill 0.6) (layers "*.Cu" "*.Mask") (remove_unused_layers no)
   (roundrect_rratio 0.15625) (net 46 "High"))
  (pad "2" thru_hole circle (at 3.6 0) (size 1.6 1.6) (drill 0.6) (layers "*.Cu" "*.Mask") (remove_unused_layers no) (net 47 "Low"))
  (pad "3" thru_hole circle (at 7.2 0) (size 1.6 1.6) (drill 0.6) (layers "*.Cu" "*.Mask") (remove_unused_layers no) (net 46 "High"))
  (pad "4" thru_hole circle (at 10.8 0) (size 1.6 1.6) (drill 0.6) (layers "*.Cu" "*.Mask") (remove_unused_layers no) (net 47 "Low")))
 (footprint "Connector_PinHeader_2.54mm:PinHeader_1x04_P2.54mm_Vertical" (layer "F.Cu") (at 36 33.5 90)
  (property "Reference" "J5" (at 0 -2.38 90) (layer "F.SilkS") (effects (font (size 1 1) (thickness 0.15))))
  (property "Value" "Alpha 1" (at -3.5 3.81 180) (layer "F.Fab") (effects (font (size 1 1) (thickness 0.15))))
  (fp_line (start -1.38 -1.38) (end 0 -1.38) (stroke (width 0.12) (type solid)) (layer "F.SilkS"))
  (fp_line (start -1.38 0) (end -1.38 -1.38) (stroke (width 0.12) (type solid)) (layer "F.SilkS"))
  (fp_line (start 1.38 1.27) (end 1.38 9) (stroke (width 0.12) (type solid)) (layer "F.SilkS"))
  (fp_line (start -1.38 1.27) (end 1.38 1.27) (stroke (width 0.12) (type solid)) (layer "F.SilkS"))
  (fp_line (start -1.38 1.27) (end -1.38 9) (stroke (width 0.12) (type solid)) (layer "F.SilkS"))
  (fp_line (start -1.38 9) (end 1.38 9) (stroke (width 0.12) (type solid)) (layer "F.SilkS"))
  (pad "1" thru_hole rect (at 0 0 90) (size 1.7 1.7) (drill 1) (layers "*.Cu" "*.Mask") (remove_unused_layers no) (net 6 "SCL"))
  (pad "2" thru_hole circle (at 0 2.54 90) (size 1.7 1.7) (drill 1) (layers "*.Cu" "*.Mask") (remove_unused_layers no) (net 7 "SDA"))
  (pad "3" thru_hole circle (at 0 5.08 90) (size 1.7 1.7) (drill 1) (layers "*.Cu" "*.Mask") (remove_unused_layers no)
   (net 8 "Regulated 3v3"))
  (pad "4" thru_hole circle (at 0 7.62 90) (size 1.7 1.7) (drill 1) (layers "*.Cu" "*.Mask") (remove_unused_layers no) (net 9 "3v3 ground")))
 (gr_rect (start 25.5 25) (end 237 156) (stroke (width 0.05) (type default)) (fill no) (layer "Edge.Cuts"))
 (segment (start 61.5 30) (end 39.5 30) (width 0.2) (layer "F.Cu") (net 6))
 (segment (start 140.373 33.438636) (end 136.934364 30) (width 0.2) (layer "F.Cu") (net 6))
 (segment (start 39.5 30) (end 36 33.5) (width 0.2) (layer "F.Cu") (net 6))
 (segment (start 109.5 30) (end 85.5 30) (width 0.2) (layer "F.Cu") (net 6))
 (segment (start 85.5 30) (end 61.5 30) (width 0.2) (layer "F.Cu") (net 6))
 (segment (start 136.934364 30) (end 109.5 30) (width 0.2) (layer "F.Cu") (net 6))
 (via (at 85.5 30) (size 0.6) (drill 0.3) (layers "F.Cu" "B.Cu") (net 6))
 (via (at 109.5 30) (size 0.6) (drill 0.3) (layers "F.Cu" "B.Cu") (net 6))
 (via (at 61.5 30) (size 0.6) (drill 0.3) (layers "F.Cu" "B.Cu") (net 6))
 (segment (start 85.5 30) (end 85.5 30.5) (width 0.2) (layer "B.Cu") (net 6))
 (segment (start 84.333333 31.666667) (end 84.333333 33.5) (width 0.2) (layer "B.Cu") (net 6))
 (segment (start 108.5 31.5) (end 108.5 33.5) (width 0.2) (layer "B.Cu") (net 6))
 (segment (start 109.5 30) (end 109.5 30.5) (width 0.2) (layer "B.Cu") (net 6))
 (segment (start 109.5 30.5) (end 108.5 31.5) (width 0.2) (layer "B.Cu") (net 6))
 (segment (start 85.5 30.5) (end 84.333333 31.666667) (width 0.2) (layer "B.Cu") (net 6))
 (segment (start 61.5 30) (end 60.166667 31.333333) (width 0.2) (layer "B.Cu") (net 6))
 (segment (start 60.166667 31.333333) (end 60.166667 33.5) (width 0.2) (layer "B.Cu") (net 6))
 (segment (start 151.545 42.763636) (end 150.533 43.775636) (width 0.2) (layer "F.Cu") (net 14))
 (segment (start 150.394 41.612636) (end 151.545 42.763636) (width 0.2) (layer "F.Cu") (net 14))
 (segment (start 150.394 39.702636) (end 150.394 41.612636) (width 0.2) (layer "F.Cu") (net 14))
 (segment (start 150.533 43.775636) (end 150.533 49.603636) (width 0.2) (layer "F.Cu") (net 14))
 (segment (start 147.74 37.048636) (end 150.394 39.702636) (width 0.2) (layer "F.Cu") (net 14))
 (segment (start 89.5 31) (end 65.206667 31) (width 0.2) (layer "F.Cu") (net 7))
 (segment (start 136.5 31) (end 113.54 31) (width 0.2) (layer "F.Cu") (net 7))
 (segment (start 89.373333 31) (end 86.873333 33.5) (width 0.2) (layer "F.Cu") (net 7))
 (segment (start 41.04 31) (end 38.54 33.5) (width 0.2) (layer "F.Cu") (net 7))
 (segment (start 142.913 31.413) (end 142.5 31) (width 0.2) (layer "F.Cu") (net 7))
 (segment (start 65.206667 31) (end 62.706667 33.5) (width 0.2) (layer "F.Cu") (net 7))
 (segment (start 113.54 31) (end 111.04 33.5) (width 0.2) (layer "F.Cu") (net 7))
 (segment (start 113.54 31) (end 89.5 31) (width 0.2) (layer "F.Cu") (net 7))
 (segment (start 65.206667 31) (end 41.04 31) (width 0.2) (layer "F.Cu") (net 7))
 (segment (start 142.913 33.438636) (end 142.913 31.413) (width 0.2) (layer "F.Cu") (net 7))
 (segment (start 89.5 31) (end 89.373333 31) (width 0.2) (layer "F.Cu") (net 7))
 (via (at 136.5 31) (size 0.6) (drill 0.3) (layers "F.Cu" "B.Cu") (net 7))
 (via (at 142.5 31) (size 0.6) (drill 0.3) (layers "F.Cu" "B.Cu") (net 7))
 (segment (start 142.5 31) (end 136.5 31) (width 0.2) (layer "B.Cu") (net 7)))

